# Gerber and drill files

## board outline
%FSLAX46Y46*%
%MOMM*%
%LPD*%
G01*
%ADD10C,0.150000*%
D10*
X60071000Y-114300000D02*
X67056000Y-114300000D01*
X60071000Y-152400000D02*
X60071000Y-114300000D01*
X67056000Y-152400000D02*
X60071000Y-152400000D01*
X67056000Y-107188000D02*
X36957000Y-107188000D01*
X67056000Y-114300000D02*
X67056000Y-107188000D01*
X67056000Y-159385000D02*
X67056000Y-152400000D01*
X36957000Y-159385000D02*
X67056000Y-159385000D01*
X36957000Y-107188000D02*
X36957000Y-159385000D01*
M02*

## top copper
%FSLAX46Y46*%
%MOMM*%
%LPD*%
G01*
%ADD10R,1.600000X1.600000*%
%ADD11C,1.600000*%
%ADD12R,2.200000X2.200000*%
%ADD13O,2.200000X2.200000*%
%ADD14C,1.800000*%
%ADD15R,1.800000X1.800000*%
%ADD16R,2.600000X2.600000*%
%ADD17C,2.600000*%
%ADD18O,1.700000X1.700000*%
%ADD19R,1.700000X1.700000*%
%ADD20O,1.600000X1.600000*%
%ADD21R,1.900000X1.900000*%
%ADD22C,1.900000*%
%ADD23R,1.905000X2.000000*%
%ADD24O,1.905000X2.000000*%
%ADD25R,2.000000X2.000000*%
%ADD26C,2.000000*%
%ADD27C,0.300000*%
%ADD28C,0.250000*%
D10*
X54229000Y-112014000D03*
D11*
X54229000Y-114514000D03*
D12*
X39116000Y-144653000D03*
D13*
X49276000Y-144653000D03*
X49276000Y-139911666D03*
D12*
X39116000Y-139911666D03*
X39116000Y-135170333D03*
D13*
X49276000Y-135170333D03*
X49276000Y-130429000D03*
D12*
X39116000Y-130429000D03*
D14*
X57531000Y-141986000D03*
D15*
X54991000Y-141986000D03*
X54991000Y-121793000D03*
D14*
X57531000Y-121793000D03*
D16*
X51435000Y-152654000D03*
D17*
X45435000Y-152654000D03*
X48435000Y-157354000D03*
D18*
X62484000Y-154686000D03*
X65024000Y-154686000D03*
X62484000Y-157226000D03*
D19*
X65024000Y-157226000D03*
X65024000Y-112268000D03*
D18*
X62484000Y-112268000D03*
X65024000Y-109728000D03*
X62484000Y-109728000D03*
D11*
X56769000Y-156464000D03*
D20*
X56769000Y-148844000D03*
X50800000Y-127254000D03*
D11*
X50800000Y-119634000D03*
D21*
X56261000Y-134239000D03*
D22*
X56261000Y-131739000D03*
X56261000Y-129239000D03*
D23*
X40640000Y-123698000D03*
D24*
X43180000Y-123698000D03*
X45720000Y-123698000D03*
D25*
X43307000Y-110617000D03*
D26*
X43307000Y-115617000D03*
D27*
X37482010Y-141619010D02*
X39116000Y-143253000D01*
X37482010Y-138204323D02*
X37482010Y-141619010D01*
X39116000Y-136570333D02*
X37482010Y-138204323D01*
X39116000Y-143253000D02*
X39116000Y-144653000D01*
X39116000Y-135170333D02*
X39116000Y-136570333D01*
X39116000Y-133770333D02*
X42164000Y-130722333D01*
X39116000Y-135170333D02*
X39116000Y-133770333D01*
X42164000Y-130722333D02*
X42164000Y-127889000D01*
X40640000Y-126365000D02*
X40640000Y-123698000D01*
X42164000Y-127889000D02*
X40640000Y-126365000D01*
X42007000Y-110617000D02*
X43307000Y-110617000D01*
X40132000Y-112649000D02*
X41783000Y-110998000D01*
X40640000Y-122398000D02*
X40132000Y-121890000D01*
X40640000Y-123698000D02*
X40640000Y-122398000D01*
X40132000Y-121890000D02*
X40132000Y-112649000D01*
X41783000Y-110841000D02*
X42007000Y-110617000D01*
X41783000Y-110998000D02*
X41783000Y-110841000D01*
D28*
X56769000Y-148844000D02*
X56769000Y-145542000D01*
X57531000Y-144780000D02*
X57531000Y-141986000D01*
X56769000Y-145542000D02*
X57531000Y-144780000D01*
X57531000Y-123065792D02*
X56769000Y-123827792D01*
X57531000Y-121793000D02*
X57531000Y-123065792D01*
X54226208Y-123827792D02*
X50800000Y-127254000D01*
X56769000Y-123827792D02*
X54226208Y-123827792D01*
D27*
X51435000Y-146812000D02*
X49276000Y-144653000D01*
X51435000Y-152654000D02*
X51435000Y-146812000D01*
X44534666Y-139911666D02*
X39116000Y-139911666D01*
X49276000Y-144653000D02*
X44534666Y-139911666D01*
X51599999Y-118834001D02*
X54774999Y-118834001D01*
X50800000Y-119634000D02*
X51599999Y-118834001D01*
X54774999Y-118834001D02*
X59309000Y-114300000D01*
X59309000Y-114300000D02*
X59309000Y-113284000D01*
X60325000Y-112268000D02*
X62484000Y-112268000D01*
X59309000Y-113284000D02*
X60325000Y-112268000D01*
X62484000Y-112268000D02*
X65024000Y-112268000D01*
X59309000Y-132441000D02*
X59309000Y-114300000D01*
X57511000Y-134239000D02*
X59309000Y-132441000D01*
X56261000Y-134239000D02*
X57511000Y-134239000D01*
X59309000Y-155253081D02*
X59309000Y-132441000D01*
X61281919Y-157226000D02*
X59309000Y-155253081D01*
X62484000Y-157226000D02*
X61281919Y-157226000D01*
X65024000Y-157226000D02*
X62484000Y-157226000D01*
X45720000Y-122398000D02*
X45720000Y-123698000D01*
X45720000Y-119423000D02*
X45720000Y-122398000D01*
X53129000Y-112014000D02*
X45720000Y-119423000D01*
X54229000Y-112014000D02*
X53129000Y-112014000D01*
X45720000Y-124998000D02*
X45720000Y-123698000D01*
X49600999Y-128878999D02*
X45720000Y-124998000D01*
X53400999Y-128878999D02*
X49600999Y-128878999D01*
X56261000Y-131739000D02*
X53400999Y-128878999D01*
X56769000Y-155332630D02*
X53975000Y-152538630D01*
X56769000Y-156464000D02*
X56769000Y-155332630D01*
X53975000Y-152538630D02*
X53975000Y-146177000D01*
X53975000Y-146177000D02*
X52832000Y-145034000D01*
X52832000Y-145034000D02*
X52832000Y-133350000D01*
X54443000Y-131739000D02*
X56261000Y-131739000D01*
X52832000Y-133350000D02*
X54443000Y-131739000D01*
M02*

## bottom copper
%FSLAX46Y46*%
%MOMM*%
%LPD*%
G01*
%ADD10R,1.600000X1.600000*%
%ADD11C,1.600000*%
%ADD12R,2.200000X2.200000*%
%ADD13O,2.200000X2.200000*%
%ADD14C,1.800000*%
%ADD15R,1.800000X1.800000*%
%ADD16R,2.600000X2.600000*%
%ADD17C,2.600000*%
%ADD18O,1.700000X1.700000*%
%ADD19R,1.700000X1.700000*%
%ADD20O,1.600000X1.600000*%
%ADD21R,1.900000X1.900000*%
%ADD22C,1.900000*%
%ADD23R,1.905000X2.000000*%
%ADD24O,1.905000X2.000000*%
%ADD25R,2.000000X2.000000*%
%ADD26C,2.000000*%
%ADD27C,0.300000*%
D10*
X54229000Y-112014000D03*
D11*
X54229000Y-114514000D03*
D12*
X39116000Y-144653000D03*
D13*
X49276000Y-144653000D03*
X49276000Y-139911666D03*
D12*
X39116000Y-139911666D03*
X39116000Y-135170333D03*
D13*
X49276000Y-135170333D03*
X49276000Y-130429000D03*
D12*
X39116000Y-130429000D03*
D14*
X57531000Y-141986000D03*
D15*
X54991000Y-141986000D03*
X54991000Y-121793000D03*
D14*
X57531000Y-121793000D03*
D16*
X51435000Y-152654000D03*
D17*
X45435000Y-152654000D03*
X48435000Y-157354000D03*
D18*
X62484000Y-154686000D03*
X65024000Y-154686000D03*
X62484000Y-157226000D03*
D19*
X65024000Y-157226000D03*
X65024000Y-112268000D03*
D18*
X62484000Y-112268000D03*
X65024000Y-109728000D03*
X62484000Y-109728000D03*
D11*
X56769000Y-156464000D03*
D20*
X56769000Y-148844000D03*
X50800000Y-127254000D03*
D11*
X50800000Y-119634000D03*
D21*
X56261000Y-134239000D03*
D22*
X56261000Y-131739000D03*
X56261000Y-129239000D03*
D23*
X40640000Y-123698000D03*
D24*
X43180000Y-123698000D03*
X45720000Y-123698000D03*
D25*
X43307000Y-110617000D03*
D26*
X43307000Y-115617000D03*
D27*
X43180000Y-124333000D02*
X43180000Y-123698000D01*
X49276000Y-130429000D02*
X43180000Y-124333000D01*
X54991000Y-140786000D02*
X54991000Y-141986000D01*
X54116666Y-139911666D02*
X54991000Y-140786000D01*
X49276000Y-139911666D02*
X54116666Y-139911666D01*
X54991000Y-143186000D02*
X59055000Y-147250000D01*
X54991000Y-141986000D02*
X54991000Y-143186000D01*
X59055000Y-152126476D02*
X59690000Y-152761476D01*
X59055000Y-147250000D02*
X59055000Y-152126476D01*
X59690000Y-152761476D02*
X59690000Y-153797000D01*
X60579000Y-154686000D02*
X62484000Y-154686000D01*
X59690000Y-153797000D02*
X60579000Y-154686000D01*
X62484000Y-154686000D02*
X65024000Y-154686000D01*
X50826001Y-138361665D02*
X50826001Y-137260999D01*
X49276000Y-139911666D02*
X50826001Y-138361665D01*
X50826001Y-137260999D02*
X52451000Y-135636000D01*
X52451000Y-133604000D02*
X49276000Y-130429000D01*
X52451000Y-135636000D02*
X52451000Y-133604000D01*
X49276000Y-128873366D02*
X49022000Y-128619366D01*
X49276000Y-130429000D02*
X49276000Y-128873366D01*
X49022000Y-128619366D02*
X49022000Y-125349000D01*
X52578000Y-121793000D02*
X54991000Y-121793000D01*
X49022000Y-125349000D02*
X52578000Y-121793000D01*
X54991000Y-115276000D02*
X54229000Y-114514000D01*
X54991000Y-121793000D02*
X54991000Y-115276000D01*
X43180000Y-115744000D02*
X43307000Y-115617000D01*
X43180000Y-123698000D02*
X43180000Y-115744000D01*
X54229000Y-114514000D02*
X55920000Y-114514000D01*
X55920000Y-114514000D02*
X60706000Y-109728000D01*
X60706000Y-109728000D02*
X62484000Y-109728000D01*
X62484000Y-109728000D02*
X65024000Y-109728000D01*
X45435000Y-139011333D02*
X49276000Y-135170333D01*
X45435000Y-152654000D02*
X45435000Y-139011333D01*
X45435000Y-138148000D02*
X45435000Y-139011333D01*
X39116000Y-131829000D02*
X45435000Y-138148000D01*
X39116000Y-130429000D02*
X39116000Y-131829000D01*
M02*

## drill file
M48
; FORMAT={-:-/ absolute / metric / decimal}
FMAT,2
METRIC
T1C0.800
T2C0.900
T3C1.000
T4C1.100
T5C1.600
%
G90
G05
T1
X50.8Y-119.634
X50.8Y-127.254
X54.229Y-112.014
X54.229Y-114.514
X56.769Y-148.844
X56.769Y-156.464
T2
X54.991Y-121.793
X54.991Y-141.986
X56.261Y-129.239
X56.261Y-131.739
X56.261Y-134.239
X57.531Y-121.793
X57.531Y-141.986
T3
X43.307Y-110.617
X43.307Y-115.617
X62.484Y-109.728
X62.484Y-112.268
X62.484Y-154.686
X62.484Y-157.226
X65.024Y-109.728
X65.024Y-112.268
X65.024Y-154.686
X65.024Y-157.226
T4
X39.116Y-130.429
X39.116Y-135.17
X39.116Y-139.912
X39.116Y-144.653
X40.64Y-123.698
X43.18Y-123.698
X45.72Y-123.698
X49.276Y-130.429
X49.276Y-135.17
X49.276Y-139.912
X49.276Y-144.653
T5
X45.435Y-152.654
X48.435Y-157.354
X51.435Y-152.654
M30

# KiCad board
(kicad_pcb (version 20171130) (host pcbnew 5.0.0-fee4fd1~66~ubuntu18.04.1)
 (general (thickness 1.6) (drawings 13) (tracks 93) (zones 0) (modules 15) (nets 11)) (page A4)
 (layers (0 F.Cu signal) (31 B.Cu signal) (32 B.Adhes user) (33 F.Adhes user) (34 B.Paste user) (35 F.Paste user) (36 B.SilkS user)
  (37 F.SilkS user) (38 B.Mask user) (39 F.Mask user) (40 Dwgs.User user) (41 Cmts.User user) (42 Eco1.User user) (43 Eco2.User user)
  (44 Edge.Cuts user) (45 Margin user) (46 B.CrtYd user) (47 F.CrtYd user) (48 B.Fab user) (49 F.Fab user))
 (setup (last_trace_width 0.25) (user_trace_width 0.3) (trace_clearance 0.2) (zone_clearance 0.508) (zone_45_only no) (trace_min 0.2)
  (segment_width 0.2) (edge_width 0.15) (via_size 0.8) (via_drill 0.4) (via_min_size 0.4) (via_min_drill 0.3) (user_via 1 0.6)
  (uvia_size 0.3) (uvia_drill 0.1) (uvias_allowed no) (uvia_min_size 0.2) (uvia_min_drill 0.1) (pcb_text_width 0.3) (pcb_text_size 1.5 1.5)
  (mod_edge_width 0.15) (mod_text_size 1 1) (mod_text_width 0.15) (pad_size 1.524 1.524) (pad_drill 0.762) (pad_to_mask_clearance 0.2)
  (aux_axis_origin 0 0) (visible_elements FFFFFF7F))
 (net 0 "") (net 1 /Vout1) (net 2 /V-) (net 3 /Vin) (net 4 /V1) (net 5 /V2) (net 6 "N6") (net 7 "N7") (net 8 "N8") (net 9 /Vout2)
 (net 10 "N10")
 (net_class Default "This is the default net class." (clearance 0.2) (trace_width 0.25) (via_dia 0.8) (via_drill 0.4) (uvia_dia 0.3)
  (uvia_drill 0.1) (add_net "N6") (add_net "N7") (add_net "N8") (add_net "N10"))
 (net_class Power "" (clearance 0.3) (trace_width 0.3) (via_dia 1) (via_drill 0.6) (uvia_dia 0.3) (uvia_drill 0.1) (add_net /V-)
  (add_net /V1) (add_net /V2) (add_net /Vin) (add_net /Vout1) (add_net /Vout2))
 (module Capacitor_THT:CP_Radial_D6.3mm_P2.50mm (layer F.Cu) (at 54.229 112.014 270)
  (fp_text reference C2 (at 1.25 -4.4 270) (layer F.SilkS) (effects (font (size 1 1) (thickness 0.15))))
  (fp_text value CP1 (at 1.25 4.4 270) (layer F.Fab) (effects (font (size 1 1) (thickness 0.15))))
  (pad 1 thru_hole rect (at 0 0 270) (size 1.6 1.6) (drill 0.8) (layers *.Cu *.Mask) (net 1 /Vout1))
  (pad 2 thru_hole circle (at 2.5 0 270) (size 1.6 1.6) (drill 0.8) (layers *.Cu *.Mask) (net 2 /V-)))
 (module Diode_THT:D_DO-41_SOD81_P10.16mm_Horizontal (layer F.Cu) (at 39.116 144.653)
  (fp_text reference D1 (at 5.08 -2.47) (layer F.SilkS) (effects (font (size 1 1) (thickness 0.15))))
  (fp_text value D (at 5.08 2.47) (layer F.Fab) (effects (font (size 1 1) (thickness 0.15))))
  (pad 1 thru_hole rect (at 0 0) (size 2.2 2.2) (drill 1.1) (layers *.Cu *.Mask) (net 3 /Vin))
  (pad 2 thru_hole oval (at 10.16 0) (size 2.2 2.2) (drill 1.1) (layers *.Cu *.Mask) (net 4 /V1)))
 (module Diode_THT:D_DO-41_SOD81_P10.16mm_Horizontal (layer F.Cu) (at 39.116 139.911666)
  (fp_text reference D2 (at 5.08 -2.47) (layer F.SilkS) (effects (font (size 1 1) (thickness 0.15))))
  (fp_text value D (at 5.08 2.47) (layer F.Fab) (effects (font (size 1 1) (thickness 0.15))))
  (pad 2 thru_hole oval (at 10.16 0) (size 2.2 2.2) (drill 1.1) (layers *.Cu *.Mask) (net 2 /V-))
  (pad 1 thru_hole rect (at 0 0) (size 2.2 2.2) (drill 1.1) (layers *.Cu *.Mask) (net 4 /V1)))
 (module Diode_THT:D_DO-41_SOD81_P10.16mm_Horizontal (layer F.Cu) (at 39.116 135.170333)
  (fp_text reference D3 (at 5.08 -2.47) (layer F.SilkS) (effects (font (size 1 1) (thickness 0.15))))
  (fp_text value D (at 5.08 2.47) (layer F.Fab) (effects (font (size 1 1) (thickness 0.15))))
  (pad 1 thru_hole rect (at 0 0) (size 2.2 2.2) (drill 1.1) (layers *.Cu *.Mask) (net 3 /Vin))
  (pad 2 thru_hole oval (at 10.16 0) (size 2.2 2.2) (drill 1.1) (layers *.Cu *.Mask) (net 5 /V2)))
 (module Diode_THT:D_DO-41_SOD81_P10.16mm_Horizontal (layer F.Cu) (at 39.116 130.429)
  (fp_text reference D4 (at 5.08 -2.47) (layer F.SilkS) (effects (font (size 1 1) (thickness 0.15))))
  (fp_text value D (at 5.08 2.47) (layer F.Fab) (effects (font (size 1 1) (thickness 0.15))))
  (pad 2 thru_hole oval (at 10.16 0) (size 2.2 2.2) (drill 1.1) (layers *.Cu *.Mask) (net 2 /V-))
  (pad 1 thru_hole rect (at 0 0) (size 2.2 2.2) (drill 1.1) (layers *.Cu *.Mask) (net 5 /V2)))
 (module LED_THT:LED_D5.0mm (layer F.Cu) (at 54.991 141.986)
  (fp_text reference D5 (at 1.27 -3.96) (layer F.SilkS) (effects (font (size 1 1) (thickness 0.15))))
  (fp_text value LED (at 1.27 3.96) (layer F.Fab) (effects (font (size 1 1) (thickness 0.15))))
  (pad 2 thru_hole circle (at 2.54 0) (size 1.8 1.8) (drill 0.9) (layers *.Cu *.Mask) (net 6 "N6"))
  (pad 1 thru_hole rect (at 0 0) (size 1.8 1.8) (drill 0.9) (layers *.Cu *.Mask) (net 2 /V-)))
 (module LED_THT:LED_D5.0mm (layer F.Cu) (at 54.991 121.793)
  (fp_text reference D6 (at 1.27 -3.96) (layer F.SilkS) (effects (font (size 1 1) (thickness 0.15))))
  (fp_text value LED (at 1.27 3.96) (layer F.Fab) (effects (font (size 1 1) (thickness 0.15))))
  (pad 1 thru_hole rect (at 0 0) (size 1.8 1.8) (drill 0.9) (layers *.Cu *.Mask) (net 2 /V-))
  (pad 2 thru_hole circle (at 2.54 0) (size 1.8 1.8) (drill 0.9) (layers *.Cu *.Mask) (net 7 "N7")))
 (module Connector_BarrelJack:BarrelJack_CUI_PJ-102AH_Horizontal (layer F.Cu) (at 51.435 152.654 270)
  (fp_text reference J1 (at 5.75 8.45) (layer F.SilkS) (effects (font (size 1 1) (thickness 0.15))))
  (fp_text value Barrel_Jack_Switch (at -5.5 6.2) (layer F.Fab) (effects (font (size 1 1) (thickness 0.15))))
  (pad 1 thru_hole rect (at 0 0 270) (size 2.6 2.6) (drill 1.6) (layers *.Cu *.Mask) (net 4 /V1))
  (pad 2 thru_hole circle (at 0 6 270) (size 2.6 2.6) (drill 1.6) (layers *.Cu *.Mask) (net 5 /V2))
  (pad 3 thru_hole circle (at 4.7 3 270) (size 2.6 2.6) (drill 1.6) (layers *.Cu *.Mask) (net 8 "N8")))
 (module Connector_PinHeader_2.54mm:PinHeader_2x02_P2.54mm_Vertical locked (layer F.Cu) (at 65.024 157.226 180)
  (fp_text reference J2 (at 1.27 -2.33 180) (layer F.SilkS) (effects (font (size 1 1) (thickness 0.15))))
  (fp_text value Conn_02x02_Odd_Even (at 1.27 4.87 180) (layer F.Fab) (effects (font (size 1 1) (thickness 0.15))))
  (pad 4 thru_hole oval (at 2.54 2.54 180) (size 1.7 1.7) (drill 1) (layers *.Cu *.Mask) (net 2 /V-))
  (pad 3 thru_hole oval (at 0 2.54 180) (size 1.7 1.7) (drill 1) (layers *.Cu *.Mask) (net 2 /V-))
  (pad 2 thru_hole oval (at 2.54 0 180) (size 1.7 1.7) (drill 1) (layers *.Cu *.Mask) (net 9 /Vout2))
  (pad 1 thru_hole rect (at 0 0 180) (size 1.7 1.7) (drill 1) (layers *.Cu *.Mask) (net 9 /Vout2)))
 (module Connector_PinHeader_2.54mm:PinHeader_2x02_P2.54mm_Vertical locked (layer F.Cu) (at 65.024 112.268 180)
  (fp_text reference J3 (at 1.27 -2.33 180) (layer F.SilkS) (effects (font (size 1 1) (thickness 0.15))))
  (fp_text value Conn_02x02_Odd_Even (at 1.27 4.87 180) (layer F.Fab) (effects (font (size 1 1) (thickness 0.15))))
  (pad 1 thru_hole rect (at 0 0 180) (size 1.7 1.7) (drill 1) (layers *.Cu *.Mask) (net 9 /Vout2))
  (pad 2 thru_hole oval (at 2.54 0 180) (size 1.7 1.7) (drill 1) (layers *.Cu *.Mask) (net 9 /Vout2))
  (pad 3 thru_hole oval (at 0 2.54 180) (size 1.7 1.7) (drill 1) (layers *.Cu *.Mask) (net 2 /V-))
  (pad 4 thru_hole oval (at 2.54 2.54 180) (size 1.7 1.7) (drill 1) (layers *.Cu *.Mask) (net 2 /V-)))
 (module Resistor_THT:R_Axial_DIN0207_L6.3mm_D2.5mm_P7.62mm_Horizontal (layer F.Cu) (at 56.769 156.464 90)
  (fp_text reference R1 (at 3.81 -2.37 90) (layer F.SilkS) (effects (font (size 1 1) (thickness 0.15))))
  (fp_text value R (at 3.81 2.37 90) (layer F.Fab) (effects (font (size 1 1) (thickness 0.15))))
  (pad 1 thru_hole circle (at 0 0 90) (size 1.6 1.6) (drill 0.8) (layers *.Cu *.Mask) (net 1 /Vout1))
  (pad 2 thru_hole oval (at 7.62 0 90) (size 1.6 1.6) (drill 0.8) (layers *.Cu *.Mask) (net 6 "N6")))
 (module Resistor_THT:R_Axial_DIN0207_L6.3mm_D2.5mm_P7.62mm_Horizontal (layer F.Cu) (at 50.8 119.634 270)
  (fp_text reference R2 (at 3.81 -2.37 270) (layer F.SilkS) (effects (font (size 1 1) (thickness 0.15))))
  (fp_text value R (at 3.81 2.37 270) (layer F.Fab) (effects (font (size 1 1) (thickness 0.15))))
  (pad 2 thru_hole oval (at 7.62 0 270) (size 1.6 1.6) (drill 0.8) (layers *.Cu *.Mask) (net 7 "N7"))
  (pad 1 thru_hole circle (at 0 0 270) (size 1.6 1.6) (drill 0.8) (layers *.Cu *.Mask) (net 9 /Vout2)))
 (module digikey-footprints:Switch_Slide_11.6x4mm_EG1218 (layer F.Cu) (at 56.261 134.239 90)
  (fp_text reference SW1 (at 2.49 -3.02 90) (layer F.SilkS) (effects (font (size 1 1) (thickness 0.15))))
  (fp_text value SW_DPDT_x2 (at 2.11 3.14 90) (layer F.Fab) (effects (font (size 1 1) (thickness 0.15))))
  (pad 1 thru_hole rect (at 0 0 90) (size 1.9 1.9) (drill 0.9) (layers *.Cu *.Mask) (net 9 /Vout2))
  (pad 2 thru_hole circle (at 2.5 0 90) (size 1.9 1.9) (drill 0.9) (layers *.Cu *.Mask) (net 1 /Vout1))
  (pad 3 thru_hole circle (at 5 0 90) (size 1.9 1.9) (drill 0.9) (layers *.Cu *.Mask) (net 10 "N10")))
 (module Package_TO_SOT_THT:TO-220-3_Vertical (layer F.Cu) (at 40.64 123.698)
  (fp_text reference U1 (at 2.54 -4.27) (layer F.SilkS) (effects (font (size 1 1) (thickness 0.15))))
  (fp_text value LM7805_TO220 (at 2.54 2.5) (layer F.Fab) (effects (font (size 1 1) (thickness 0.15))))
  (pad 1 thru_hole rect (at 0 0) (size 1.905 2) (drill 1.1) (layers *.Cu *.Mask) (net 3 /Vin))
  (pad 2 thru_hole oval (at 2.54 0) (size 1.905 2) (drill 1.1) (layers *.Cu *.Mask) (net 2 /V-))
  (pad 3 thru_hole oval (at 5.08 0) (size 1.905 2) (drill 1.1) (layers *.Cu *.Mask) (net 1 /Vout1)))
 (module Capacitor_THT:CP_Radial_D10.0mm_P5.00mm (layer F.Cu) (at 43.307 110.617 270)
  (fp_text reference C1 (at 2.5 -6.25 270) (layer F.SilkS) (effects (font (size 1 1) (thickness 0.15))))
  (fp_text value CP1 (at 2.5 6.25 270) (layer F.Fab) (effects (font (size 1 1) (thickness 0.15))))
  (pad 1 thru_hole rect (at 0 0 270) (size 2 2) (drill 1) (layers *.Cu *.Mask) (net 3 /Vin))
  (pad 2 thru_hole circle (at 5 0 270) (size 2 2) (drill 1) (layers *.Cu *.Mask) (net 2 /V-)))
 (gr_line (start 60.071 114.3) (end 67.056 114.3) (layer Edge.Cuts) (width 0.15))
 (gr_line (start 60.071 152.4) (end 60.071 114.3) (layer Edge.Cuts) (width 0.15))
 (gr_line (start 67.056 152.4) (end 60.071 152.4) (layer Edge.Cuts) (width 0.15))
 (gr_line (start 67.056 107.188) (end 36.957 107.188) (layer Edge.Cuts) (width 0.15))
 (gr_line (start 67.056 114.3) (end 67.056 107.188) (layer Edge.Cuts) (width 0.15))
 (gr_line (start 67.056 159.385) (end 67.056 152.4) (layer Edge.Cuts) (width 0.15))
 (gr_line (start 36.957 159.385) (end 67.056 159.385) (layer Edge.Cuts) (width 0.15))
 (gr_line (start 36.957 107.188) (end 36.957 159.385) (layer Edge.Cuts) (width 0.15))
 (segment (start 37.48201 141.61901) (end 39.116 143.253) (width 0.3) (layer F.Cu) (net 3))
 (segment (start 37.48201 138.204323) (end 37.48201 141.61901) (width 0.3) (layer F.Cu) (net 3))
 (segment (start 39.116 136.570333) (end 37.48201 138.204323) (width 0.3) (layer F.Cu) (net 3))
 (segment (start 39.116 143.253) (end 39.116 144.653) (width 0.3) (layer F.Cu) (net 3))
 (segment (start 39.116 135.170333) (end 39.116 136.570333) (width 0.3) (layer F.Cu) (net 3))
 (segment (start 39.116 133.770333) (end 42.164 130.722333) (width 0.3) (layer F.Cu) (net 3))
 (segment (start 39.116 135.170333) (end 39.116 133.770333) (width 0.3) (layer F.Cu) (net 3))
 (segment (start 42.164 130.722333) (end 42.164 127.889) (width 0.3) (layer F.Cu) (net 3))
 (segment (start 40.64 126.365) (end 40.64 123.698) (width 0.3) (layer F.Cu) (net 3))
 (segment (start 42.164 127.889) (end 40.64 126.365) (width 0.3) (layer F.Cu) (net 3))
 (segment (start 42.007 110.617) (end 43.307 110.617) (width 0.3) (layer F.Cu) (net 3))
 (segment (start 40.132 112.649) (end 41.783 110.998) (width 0.3) (layer F.Cu) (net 3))
 (segment (start 40.64 122.398) (end 40.132 121.89) (width 0.3) (layer F.Cu) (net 3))
 (segment (start 40.64 123.698) (end 40.64 122.398) (width 0.3) (layer F.Cu) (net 3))
 (segment (start 40.132 121.89) (end 40.132 112.649) (width 0.3) (layer F.Cu) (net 3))
 (segment (start 41.783 110.841) (end 42.007 110.617) (width 0.3) (layer F.Cu) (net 3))
 (segment (start 41.783 110.998) (end 41.783 110.841) (width 0.3) (layer F.Cu) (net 3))
 (segment (start 43.18 124.333) (end 43.18 123.698) (width 0.3) (layer B.Cu) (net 2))
 (segment (start 49.276 130.429) (end 43.18 124.333) (width 0.3) (layer B.Cu) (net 2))
 (segment (start 54.991 140.786) (end 54.991 141.986) (width 0.3) (layer B.Cu) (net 2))
 (segment (start 54.116666 139.911666) (end 54.991 140.786) (width 0.3) (layer B.Cu) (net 2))
 (segment (start 49.276 139.911666) (end 54.116666 139.911666) (width 0.3) (layer B.Cu) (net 2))
 (segment (start 54.991 143.186) (end 59.055 147.25) (width 0.3) (layer B.Cu) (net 2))
 (segment (start 54.991 141.986) (end 54.991 143.186) (width 0.3) (layer B.Cu) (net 2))
 (segment (start 59.055 152.126476) (end 59.69 152.761476) (width 0.3) (layer B.Cu) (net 2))
 (segment (start 59.055 147.25) (end 59.055 152.126476) (width 0.3) (layer B.Cu) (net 2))
 (segment (start 59.69 152.761476) (end 59.69 153.797) (width 0.3) (layer B.Cu) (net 2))
 (segment (start 60.579 154.686) (end 62.484 154.686) (width 0.3) (layer B.Cu) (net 2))
 (segment (start 59.69 153.797) (end 60.579 154.686) (width 0.3) (layer B.Cu) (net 2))
 (segment (start 62.484 154.686) (end 65.024 154.686) (width 0.3) (layer B.Cu) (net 2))
 (segment (start 50.826001 138.361665) (end 50.826001 137.260999) (width 0.3) (layer B.Cu) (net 2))
 (segment (start 49.276 139.911666) (end 50.826001 138.361665) (width 0.3) (layer B.Cu) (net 2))
 (segment (start 50.826001 137.260999) (end 52.451 135.636) (width 0.3) (layer B.Cu) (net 2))
 (segment (start 52.451 133.604) (end 49.276 130.429) (width 0.3) (layer B.Cu) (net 2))
 (segment (start 52.451 135.636) (end 52.451 133.604) (width 0.3) (layer B.Cu) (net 2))
 (segment (start 49.276 128.873366) (end 49.022 128.619366) (width 0.3) (layer B.Cu) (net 2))
 (segment (start 49.276 130.429) (end 49.276 128.873366) (width 0.3) (layer B.Cu) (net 2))
 (segment (start 49.022 128.619366) (end 49.022 125.349) (width 0.3) (layer B.Cu) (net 2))
 (segment (start 52.578 121.793) (end 54.991 121.793) (width 0.3) (layer B.Cu) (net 2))
 (segment (start 49.022 125.349) (end 52.578 121.793) (width 0.3) (layer B.Cu) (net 2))
 (segment (start 54.991 115.276) (end 54.229 114.514) (width 0.3) (layer B.Cu) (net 2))
 (segment (start 54.991 121.793) (end 54.991 115.276) (width 0.3) (layer B.Cu) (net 2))
 (segment (start 43.18 115.744) (end 43.307 115.617) (width 0.3) (layer B.Cu) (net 2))
 (segment (start 43.18 123.698) (end 43.18 115.744) (width 0.3) (layer B.Cu) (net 2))
 (segment (start 54.229 114.514) (end 55.92 114.514) (width 0.3) (layer B.Cu) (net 2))
 (segment (start 55.92 114.514) (end 60.706 109.728) (width 0.3) (layer B.Cu) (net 2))
 (segment (start 60.706 109.728) (end 62.484 109.728) (width 0.3) (layer B.Cu) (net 2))
 (segment (start 62.484 109.728) (end 65.024 109.728) (width 0.3) (layer B.Cu) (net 2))
 (segment (start 56.769 148.844) (end 56.769 145.542) (width 0.25) (layer F.Cu) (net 6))
 (segment (start 57.531 144.78) (end 57.531 141.986) (width 0.25) (layer F.Cu) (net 6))
 (segment (start 56.769 145.542) (end 57.531 144.78) (width 0.25) (layer F.Cu) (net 6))
 (segment (start 57.531 123.065792) (end 56.769 123.827792) (width 0.25) (layer F.Cu) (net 7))
 (segment (start 57.531 121.793) (end 57.531 123.065792) (width 0.25) (layer F.Cu) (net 7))
 (segment (start 54.226208 123.827792) (end 50.8 127.254) (width 0.25) (layer F.Cu) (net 7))
 (segment (start 56.769 123.827792) (end 54.226208 123.827792) (width 0.25) (layer F.Cu) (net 7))
 (segment (start 51.435 146.812) (end 49.276 144.653) (width 0.3) (layer F.Cu) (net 4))
 (segment (start 51.435 152.654) (end 51.435 146.812) (width 0.3) (layer F.Cu) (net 4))
 (segment (start 44.534666 139.911666) (end 39.116 139.911666) (width 0.3) (layer F.Cu) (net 4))
 (segment (start 49.276 144.653) (end 44.534666 139.911666) (width 0.3) (layer F.Cu) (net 4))
 (segment (start 45.435 139.011333) (end 49.276 135.170333) (width 0.3) (layer B.Cu) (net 5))
 (segment (start 45.435 152.654) (end 45.435 139.011333) (width 0.3) (layer B.Cu) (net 5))
 (segment (start 45.435 138.148) (end 45.435 139.011333) (width 0.3) (layer B.Cu) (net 5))
 (segment (start 39.116 131.829) (end 45.435 138.148) (width 0.3) (layer B.Cu) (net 5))
 (segment (start 39.116 130.429) (end 39.116 131.829) (width 0.3) (layer B.Cu) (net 5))
 (segment (start 51.599999 118.834001) (end 54.774999 118.834001) (width 0.3) (layer F.Cu) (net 9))
 (segment (start 50.8 119.634) (end 51.599999 118.834001) (width 0.3) (layer F.Cu) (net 9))
 (segment (start 54.774999 118.834001) (end 59.309 114.3) (width 0.3) (layer F.Cu) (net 9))
 (segment (start 59.309 114.3) (end 59.309 113.284) (width 0.3) (layer F.Cu) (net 9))
 (segment (start 60.325 112.268) (end 62.484 112.268) (width 0.3) (layer F.Cu) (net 9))
 (segment (start 59.309 113.284) (end 60.325 112.268) (width 0.3) (layer F.Cu) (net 9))
 (segment (start 62.484 112.268) (end 65.024 112.268) (width 0.3) (layer F.Cu) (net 9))
 (segment (start 59.309 132.441) (end 59.309 114.3) (width 0.3) (layer F.Cu) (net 9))
 (segment (start 57.511 134.239) (end 59.309 132.441) (width 0.3) (layer F.Cu) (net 9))
 (segment (start 56.261 134.239) (end 57.511 134.239) (width 0.3) (layer F.Cu) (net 9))
 (segment (start 59.309 155.253081) (end 59.309 132.441) (width 0.3) (layer F.Cu) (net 9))
 (segment (start 61.281919 157.226) (end 59.309 155.253081) (width 0.3) (layer F.Cu) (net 9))
 (segment (start 62.484 157.226) (end 61.281919 157.226) (width 0.3) (layer F.Cu) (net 9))
 (segment (start 65.024 157.226) (end 62.484 157.226) (width 0.3) (layer F.Cu) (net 9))
 (segment (start 45.72 122.398) (end 45.72 123.698) (width 0.3) (layer F.Cu) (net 1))
 (segment (start 45.72 119.423) (end 45.72 122.398) (width 0.3) (layer F.Cu) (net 1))
 (segment (start 53.129 112.014) (end 45.72 119.423) (width 0.3) (layer F.Cu) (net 1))
 (segment (start 54.229 112.014) (end 53.129 112.014) (width 0.3) (layer F.Cu) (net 1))
 (segment (start 45.72 124.998) (end 45.72 123.698) (width 0.3) (layer F.Cu) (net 1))
 (segment (start 49.600999 128.878999) (end 45.72 124.998) (width 0.3) (layer F.Cu) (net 1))
 (segment (start 53.400999 128.878999) (end 49.600999 128.878999) (width 0.3) (layer F.Cu) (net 1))
 (segment (start 56.261 131.739) (end 53.400999 128.878999) (width 0.3) (layer F.Cu) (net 1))
 (segment (start 56.769 155.33263) (end 53.975 152.53863) (width 0.3) (layer F.Cu) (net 1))
 (segment (start 56.769 156.464) (end 56.769 155.33263) (width 0.3) (layer F.Cu) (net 1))
 (segment (start 53.975 152.53863) (end 53.975 146.177) (width 0.3) (layer F.Cu) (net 1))
 (segment (start 53.975 146.177) (end 52.832 145.034) (width 0.3) (layer F.Cu) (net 1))
 (segment (start 52.832 145.034) (end 52.832 133.35) (width 0.3) (layer F.Cu) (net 1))
 (segment (start 54.443 131.739) (end 56.261 131.739) (width 0.3) (layer F.Cu) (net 1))
 (segment (start 52.832 133.35) (end 54.443 131.739) (width 0.3) (layer F.Cu) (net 1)))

